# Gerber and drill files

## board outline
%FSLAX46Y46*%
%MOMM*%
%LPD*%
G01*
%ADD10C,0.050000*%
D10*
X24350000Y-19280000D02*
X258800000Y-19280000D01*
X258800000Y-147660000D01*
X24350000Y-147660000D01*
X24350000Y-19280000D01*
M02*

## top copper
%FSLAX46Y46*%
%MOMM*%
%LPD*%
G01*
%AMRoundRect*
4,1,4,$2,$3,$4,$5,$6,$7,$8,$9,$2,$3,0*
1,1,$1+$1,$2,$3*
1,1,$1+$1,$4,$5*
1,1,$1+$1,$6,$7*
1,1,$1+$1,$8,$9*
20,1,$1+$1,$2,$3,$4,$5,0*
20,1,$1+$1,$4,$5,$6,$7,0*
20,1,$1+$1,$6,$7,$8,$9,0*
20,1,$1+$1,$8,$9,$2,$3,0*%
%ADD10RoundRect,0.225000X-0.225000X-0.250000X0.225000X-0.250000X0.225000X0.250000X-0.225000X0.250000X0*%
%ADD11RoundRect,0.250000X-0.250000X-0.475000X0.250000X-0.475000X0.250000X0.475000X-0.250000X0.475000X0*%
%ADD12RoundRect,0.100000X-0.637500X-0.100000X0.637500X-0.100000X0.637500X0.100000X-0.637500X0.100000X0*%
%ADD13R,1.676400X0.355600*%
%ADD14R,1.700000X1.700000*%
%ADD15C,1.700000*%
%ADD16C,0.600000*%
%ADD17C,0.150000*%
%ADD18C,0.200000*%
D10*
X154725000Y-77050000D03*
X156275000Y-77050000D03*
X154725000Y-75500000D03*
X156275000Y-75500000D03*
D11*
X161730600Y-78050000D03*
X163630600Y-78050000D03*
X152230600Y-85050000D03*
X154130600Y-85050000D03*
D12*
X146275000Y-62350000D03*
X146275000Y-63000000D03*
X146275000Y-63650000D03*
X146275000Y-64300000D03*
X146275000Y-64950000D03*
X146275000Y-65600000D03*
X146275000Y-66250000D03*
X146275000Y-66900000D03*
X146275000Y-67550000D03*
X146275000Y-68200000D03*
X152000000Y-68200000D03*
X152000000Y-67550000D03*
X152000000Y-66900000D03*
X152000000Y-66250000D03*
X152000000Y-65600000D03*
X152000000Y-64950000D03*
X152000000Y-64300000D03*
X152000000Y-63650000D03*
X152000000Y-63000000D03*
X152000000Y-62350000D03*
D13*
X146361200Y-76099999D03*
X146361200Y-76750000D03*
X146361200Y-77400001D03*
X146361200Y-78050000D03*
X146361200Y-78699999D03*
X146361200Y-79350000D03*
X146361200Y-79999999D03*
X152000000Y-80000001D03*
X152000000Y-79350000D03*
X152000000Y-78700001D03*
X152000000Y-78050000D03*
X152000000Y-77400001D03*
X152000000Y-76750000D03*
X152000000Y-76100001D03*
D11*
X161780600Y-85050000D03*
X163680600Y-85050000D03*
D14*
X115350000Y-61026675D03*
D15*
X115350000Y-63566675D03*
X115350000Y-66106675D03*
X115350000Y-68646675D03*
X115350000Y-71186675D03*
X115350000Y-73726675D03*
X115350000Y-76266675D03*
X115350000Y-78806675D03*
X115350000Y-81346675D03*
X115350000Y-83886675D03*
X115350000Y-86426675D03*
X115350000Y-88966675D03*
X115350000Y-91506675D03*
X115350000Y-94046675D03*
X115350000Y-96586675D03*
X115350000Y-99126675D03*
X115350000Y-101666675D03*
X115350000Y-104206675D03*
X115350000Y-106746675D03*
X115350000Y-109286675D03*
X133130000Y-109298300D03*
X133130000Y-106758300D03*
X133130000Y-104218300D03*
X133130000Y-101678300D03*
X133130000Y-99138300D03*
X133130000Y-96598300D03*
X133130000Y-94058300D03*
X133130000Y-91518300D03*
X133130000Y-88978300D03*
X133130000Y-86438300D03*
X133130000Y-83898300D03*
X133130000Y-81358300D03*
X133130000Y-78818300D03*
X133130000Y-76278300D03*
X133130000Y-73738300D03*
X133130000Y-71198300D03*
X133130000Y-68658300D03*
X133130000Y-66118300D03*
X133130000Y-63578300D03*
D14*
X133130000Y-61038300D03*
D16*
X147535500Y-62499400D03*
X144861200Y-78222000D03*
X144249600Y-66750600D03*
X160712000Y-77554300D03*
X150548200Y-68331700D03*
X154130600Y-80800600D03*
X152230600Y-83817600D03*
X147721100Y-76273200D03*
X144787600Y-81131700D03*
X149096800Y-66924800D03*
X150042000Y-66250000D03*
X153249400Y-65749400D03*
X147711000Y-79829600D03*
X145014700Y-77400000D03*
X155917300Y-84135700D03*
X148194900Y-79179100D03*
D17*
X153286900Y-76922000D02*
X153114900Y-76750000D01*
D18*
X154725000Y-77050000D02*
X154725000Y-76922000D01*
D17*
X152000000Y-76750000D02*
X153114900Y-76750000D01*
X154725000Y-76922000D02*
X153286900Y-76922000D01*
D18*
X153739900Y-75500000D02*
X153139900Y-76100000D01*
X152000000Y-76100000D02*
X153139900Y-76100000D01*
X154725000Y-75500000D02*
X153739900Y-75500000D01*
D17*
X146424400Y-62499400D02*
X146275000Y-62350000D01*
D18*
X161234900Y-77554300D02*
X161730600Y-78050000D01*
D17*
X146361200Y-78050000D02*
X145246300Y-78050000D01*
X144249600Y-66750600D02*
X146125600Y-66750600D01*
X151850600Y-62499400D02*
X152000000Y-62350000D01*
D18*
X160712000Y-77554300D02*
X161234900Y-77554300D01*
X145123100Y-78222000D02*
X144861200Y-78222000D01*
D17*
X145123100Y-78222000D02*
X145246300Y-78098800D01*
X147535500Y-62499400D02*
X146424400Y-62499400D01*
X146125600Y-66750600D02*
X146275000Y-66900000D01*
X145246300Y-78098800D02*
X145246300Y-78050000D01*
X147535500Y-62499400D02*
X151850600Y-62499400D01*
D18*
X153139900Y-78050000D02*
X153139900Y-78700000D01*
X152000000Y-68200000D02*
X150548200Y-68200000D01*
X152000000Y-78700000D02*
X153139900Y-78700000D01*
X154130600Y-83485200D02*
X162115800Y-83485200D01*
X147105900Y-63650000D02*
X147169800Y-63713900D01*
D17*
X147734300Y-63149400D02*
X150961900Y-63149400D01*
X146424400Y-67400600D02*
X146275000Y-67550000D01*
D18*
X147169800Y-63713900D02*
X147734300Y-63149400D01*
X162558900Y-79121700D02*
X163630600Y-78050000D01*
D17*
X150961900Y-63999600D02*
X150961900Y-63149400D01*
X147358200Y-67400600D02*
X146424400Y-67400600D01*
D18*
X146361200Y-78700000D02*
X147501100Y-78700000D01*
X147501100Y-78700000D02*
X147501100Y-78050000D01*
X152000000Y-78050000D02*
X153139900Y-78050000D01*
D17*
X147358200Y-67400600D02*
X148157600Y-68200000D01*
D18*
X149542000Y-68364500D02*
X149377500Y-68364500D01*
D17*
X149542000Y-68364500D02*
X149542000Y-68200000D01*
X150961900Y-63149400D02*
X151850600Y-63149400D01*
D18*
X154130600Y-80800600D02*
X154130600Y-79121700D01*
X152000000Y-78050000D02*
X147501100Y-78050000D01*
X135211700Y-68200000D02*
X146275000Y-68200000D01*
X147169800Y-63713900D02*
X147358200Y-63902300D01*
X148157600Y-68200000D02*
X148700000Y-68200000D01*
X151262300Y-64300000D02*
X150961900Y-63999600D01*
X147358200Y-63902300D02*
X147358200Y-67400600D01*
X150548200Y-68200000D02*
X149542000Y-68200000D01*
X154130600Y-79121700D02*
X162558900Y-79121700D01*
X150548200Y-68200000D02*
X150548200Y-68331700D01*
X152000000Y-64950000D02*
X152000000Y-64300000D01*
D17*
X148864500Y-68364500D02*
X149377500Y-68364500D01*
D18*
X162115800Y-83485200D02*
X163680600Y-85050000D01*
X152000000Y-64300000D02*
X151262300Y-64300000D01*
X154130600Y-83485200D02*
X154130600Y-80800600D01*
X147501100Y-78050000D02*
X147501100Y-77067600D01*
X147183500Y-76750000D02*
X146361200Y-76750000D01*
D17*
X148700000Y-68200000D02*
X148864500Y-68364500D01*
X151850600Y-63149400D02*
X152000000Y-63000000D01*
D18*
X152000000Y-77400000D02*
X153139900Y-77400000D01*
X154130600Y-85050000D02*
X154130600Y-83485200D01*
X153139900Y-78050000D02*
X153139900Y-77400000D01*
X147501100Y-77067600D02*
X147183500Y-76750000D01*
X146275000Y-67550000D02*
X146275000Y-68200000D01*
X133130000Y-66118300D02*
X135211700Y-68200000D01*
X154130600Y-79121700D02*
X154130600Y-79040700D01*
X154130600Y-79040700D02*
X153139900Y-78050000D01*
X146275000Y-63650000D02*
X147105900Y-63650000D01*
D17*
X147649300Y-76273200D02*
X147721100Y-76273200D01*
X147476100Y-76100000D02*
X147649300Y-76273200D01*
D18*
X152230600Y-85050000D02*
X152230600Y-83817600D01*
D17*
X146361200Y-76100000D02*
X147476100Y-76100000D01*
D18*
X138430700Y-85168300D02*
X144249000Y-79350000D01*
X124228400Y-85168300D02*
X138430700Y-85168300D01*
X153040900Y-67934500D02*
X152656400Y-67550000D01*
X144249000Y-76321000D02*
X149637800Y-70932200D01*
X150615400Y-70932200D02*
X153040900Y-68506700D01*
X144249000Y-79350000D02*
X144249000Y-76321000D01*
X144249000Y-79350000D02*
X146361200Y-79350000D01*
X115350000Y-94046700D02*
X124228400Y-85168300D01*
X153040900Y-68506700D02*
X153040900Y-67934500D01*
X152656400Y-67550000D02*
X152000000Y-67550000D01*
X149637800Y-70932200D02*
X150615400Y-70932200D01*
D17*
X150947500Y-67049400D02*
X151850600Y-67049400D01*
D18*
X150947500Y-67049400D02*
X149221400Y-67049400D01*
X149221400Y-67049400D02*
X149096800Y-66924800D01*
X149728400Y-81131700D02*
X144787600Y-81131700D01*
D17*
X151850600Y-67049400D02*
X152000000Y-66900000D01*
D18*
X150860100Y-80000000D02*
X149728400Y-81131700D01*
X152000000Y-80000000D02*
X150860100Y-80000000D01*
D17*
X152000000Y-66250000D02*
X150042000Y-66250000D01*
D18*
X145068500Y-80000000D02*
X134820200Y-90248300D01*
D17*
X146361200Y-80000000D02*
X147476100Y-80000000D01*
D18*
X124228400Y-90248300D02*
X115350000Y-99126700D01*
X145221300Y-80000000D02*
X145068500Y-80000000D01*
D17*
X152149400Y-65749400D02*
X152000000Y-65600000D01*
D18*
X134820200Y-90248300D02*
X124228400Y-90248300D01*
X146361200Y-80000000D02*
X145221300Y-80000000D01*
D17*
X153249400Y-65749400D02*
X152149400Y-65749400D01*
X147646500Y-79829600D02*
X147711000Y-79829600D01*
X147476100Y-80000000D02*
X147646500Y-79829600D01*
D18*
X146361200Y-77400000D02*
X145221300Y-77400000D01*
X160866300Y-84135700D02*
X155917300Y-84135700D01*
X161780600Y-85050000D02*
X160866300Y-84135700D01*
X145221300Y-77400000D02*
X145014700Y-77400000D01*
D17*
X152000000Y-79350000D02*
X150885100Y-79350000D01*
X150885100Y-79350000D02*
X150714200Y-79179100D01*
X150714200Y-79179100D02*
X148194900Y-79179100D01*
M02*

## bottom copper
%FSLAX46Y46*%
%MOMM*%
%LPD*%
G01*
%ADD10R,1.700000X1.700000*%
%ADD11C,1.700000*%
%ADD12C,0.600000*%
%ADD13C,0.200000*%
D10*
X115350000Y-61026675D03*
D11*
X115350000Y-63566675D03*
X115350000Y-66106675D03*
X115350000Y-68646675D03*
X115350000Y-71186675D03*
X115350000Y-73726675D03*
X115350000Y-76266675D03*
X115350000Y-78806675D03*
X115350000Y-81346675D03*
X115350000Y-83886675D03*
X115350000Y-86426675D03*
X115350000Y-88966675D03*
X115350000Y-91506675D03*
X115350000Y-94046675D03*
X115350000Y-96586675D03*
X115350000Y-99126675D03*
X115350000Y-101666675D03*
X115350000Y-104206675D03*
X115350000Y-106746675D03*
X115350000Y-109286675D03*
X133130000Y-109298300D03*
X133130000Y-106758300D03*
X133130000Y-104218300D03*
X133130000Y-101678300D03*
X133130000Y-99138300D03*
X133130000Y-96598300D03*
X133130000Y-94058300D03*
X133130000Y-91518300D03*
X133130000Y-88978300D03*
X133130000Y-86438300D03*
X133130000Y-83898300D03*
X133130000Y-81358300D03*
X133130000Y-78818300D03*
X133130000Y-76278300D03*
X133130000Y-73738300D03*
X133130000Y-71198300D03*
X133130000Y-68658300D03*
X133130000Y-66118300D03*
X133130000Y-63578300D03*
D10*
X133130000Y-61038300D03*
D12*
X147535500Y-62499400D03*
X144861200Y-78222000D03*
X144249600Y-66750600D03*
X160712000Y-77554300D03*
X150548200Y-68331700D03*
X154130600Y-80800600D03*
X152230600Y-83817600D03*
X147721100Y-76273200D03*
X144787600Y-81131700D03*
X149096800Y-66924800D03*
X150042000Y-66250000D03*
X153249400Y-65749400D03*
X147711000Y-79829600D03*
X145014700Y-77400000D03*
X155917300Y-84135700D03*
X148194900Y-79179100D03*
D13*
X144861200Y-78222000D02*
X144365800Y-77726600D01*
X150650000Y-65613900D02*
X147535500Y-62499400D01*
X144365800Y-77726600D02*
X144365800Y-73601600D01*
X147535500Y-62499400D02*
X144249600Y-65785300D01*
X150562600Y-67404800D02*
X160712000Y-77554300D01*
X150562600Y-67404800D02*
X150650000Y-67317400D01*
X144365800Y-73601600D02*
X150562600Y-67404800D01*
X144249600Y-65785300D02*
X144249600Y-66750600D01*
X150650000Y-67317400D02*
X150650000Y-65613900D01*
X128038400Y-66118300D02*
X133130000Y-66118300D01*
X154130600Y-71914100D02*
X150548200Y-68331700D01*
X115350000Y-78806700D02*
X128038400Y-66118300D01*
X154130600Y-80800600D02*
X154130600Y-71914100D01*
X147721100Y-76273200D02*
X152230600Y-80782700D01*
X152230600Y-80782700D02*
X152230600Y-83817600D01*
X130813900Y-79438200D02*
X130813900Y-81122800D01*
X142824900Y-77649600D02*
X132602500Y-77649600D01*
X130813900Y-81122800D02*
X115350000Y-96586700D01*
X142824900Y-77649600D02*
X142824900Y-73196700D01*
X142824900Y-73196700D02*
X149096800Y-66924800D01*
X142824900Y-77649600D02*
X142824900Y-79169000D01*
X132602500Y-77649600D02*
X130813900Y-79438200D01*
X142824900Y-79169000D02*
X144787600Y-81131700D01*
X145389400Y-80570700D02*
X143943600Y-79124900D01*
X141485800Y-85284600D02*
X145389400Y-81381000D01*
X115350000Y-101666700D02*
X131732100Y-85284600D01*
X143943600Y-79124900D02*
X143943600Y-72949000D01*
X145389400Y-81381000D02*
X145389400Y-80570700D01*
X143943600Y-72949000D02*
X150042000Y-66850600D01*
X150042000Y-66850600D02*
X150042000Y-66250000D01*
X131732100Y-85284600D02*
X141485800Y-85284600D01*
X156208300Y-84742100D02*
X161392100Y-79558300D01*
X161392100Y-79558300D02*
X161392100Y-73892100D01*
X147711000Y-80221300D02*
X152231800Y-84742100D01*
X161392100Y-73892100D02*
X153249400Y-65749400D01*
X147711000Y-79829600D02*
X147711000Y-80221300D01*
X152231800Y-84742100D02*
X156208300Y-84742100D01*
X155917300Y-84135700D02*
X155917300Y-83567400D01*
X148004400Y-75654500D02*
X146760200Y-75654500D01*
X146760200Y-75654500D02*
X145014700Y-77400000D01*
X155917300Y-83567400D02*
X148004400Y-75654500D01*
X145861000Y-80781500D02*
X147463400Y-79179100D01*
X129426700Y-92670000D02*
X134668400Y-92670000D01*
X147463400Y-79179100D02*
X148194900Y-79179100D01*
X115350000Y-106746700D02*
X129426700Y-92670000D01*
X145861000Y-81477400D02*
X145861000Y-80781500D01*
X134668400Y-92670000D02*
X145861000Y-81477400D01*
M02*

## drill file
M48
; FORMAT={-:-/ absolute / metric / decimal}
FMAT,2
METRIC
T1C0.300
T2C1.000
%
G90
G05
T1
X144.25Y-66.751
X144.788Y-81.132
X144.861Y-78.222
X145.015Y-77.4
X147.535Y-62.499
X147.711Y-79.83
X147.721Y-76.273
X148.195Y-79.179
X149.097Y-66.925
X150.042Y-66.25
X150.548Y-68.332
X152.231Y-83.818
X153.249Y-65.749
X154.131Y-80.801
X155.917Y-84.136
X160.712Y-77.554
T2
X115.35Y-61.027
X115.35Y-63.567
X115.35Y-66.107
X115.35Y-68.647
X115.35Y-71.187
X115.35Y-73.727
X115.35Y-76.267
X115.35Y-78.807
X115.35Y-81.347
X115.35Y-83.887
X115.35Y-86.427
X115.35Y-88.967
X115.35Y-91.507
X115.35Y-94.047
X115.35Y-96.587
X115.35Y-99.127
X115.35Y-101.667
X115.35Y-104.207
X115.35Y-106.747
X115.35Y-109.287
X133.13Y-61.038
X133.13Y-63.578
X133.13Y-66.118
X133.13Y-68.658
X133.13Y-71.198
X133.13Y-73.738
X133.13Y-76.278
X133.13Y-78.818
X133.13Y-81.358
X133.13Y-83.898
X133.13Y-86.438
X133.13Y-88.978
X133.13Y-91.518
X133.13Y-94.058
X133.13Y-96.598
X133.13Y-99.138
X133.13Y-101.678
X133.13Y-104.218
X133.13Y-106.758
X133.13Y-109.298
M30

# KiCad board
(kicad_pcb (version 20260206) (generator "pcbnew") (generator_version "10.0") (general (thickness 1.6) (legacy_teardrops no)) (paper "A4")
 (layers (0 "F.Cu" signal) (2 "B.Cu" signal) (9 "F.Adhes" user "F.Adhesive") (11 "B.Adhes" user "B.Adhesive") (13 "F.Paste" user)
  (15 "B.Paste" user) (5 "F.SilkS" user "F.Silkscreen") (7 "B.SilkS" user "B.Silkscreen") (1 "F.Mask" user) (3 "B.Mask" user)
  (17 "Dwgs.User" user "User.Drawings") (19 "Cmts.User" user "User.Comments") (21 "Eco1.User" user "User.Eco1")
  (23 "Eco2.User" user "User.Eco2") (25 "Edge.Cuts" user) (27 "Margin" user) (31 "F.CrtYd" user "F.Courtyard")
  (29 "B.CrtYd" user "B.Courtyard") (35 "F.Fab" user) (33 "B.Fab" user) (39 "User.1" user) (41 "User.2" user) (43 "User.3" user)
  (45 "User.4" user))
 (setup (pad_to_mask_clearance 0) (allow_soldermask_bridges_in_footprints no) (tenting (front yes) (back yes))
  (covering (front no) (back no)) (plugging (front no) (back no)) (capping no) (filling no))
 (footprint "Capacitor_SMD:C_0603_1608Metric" (layer "F.Cu") (at 155.5 77.05)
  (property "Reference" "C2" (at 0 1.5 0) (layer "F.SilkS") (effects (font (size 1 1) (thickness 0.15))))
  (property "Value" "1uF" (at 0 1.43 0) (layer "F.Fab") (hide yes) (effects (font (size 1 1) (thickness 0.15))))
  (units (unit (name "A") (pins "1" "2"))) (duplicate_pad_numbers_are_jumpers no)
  (pad "1" smd roundrect (at -0.775 0) (size 0.9 0.95) (layers "F.Cu" "F.Mask" "F.Paste") (roundrect_rratio 0.25) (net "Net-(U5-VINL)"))
  (pad "2" smd roundrect (at 0.775 0) (size 0.9 0.95) (layers "F.Cu" "F.Mask" "F.Paste") (roundrect_rratio 0.25) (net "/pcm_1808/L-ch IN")))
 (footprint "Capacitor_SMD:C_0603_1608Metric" (layer "F.Cu") (at 155.5 75.5)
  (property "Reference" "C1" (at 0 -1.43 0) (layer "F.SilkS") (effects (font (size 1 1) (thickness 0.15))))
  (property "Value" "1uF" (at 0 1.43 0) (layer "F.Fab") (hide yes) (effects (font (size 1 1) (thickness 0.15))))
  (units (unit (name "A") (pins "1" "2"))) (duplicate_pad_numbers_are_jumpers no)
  (pad "1" smd roundrect (at -0.775 0) (size 0.9 0.95) (layers "F.Cu" "F.Mask" "F.Paste") (roundrect_rratio 0.25) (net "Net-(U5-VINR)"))
  (pad "2" smd roundrect (at 0.775 0) (size 0.9 0.95) (layers "F.Cu" "F.Mask" "F.Paste") (roundrect_rratio 0.25) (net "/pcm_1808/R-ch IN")))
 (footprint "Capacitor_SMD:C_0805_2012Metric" (layer "F.Cu") (at 162.6806 78.05)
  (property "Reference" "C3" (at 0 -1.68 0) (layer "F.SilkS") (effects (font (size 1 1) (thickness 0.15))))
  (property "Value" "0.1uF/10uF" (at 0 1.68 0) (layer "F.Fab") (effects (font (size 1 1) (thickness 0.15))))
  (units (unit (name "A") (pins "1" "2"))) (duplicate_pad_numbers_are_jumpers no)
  (pad "1" smd roundrect (at -0.95 0) (size 1 1.45) (layers "F.Cu" "F.Mask" "F.Paste") (roundrect_rratio 0.25) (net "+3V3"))
  (pad "2" smd roundrect (at 0.95 0) (size 1 1.45) (layers "F.Cu" "F.Mask" "F.Paste") (roundrect_rratio 0.25) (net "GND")))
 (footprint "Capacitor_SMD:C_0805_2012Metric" (layer "F.Cu") (at 153.1806 85.05)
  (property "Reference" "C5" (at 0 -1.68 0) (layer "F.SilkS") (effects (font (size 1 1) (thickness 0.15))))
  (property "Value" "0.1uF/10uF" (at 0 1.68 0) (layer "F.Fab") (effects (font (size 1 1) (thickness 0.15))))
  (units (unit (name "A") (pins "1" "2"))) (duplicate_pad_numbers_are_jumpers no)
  (pad "1" smd roundrect (at -0.95 0) (size 1 1.45) (layers "F.Cu" "F.Mask" "F.Paste") (roundrect_rratio 0.25) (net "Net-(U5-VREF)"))
  (pad "2" smd roundrect (at 0.95 0) (size 1 1.45) (layers "F.Cu" "F.Mask" "F.Paste") (roundrect_rratio 0.25) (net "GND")))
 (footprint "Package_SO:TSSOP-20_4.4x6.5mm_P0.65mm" (layer "F.Cu") (at 149.1375 65.275)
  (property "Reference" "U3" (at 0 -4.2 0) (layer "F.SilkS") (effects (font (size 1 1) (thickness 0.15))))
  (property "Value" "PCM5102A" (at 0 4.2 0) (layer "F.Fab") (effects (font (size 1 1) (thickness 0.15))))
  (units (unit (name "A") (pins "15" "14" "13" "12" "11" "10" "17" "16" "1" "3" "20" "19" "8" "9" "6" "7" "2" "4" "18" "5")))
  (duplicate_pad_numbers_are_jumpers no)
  (pad "1" smd roundrect (at -2.8625 -2.925) (size 1.475 0.4) (layers "F.Cu" "F.Mask" "F.Paste") (roundrect_rratio 0.25) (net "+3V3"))
  (pad "2" smd roundrect (at -2.8625 -2.275) (size 1.475 0.4) (layers "F.Cu" "F.Mask" "F.Paste") (roundrect_rratio 0.25)
   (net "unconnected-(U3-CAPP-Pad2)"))
  (pad "3" smd roundrect (at -2.8625 -1.625) (size 1.475 0.4) (layers "F.Cu" "F.Mask" "F.Paste") (roundrect_rratio 0.25) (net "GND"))
  (pad "4" smd roundrect (at -2.8625 -0.975) (size 1.475 0.4) (layers "F.Cu" "F.Mask" "F.Paste") (roundrect_rratio 0.25)
   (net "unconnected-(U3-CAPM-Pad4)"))
  (pad "5" smd roundrect (at -2.8625 -0.325) (size 1.475 0.4) (layers "F.Cu" "F.Mask" "F.Paste") (roundrect_rratio 0.25) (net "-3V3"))
  (pad "6" smd roundrect (at -2.8625 0.325) (size 1.475 0.4) (layers "F.Cu" "F.Mask" "F.Paste") (roundrect_rratio 0.25)
   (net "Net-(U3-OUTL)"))
  (pad "7" smd roundrect (at -2.8625 0.975) (size 1.475 0.4) (layers "F.Cu" "F.Mask" "F.Paste") (roundrect_rratio 0.25)
   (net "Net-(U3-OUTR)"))
  (pad "8" smd roundrect (at -2.8625 1.625) (size 1.475 0.4) (layers "F.Cu" "F.Mask" "F.Paste") (roundrect_rratio 0.25) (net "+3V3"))
  (pad "9" smd roundrect (at -2.8625 2.275) (size 1.475 0.4) (layers "F.Cu" "F.Mask" "F.Paste") (roundrect_rratio 0.25) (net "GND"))
  (pad "10" smd roundrect (at -2.8625 2.925) (size 1.475 0.4) (layers "F.Cu" "F.Mask" "F.Paste") (roundrect_rratio 0.25) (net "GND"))
  (pad "11" smd roundrect (at 2.8625 2.925) (size 1.475 0.4) (layers "F.Cu" "F.Mask" "F.Paste") (roundrect_rratio 0.25) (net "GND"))
  (pad "12" smd roundrect (at 2.8625 2.275) (size 1.475 0.4) (layers "F.Cu" "F.Mask" "F.Paste") (roundrect_rratio 0.25) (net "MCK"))
  (pad "13" smd roundrect (at 2.8625 1.625) (size 1.475 0.4) (layers "F.Cu" "F.Mask" "F.Paste") (roundrect_rratio 0.25) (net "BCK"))
  (pad "14" smd roundrect (at 2.8625 0.975) (size 1.475 0.4) (layers "F.Cu" "F.Mask" "F.Paste") (roundrect_rratio 0.25) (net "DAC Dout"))
  (pad "15" smd roundrect (at 2.8625 0.325) (size 1.475 0.4) (layers "F.Cu" "F.Mask" "F.Paste") (roundrect_rratio 0.25) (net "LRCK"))
  (pad "16" smd roundrect (at 2.8625 -0.325) (size 1.475 0.4) (layers "F.Cu" "F.Mask" "F.Paste") (roundrect_rratio 0.25) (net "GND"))
  (pad "17" smd roundrect (at 2.8625 -0.975) (size 1.475 0.4) (layers "F.Cu" "F.Mask" "F.Paste") (roundrect_rratio 0.25) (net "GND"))
  (pad "18" smd roundrect (at 2.8625 -1.625) (size 1.475 0.4) (layers "F.Cu" "F.Mask" "F.Paste") (roundrect_rratio 0.25)
   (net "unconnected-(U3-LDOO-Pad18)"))
  (pad "19" smd roundrect (at 2.8625 -2.275) (size 1.475 0.4) (layers "F.Cu" "F.Mask" "F.Paste") (roundrect_rratio 0.25) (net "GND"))
  (pad "20" smd roundrect (at 2.8625 -2.925) (size 1.475 0.4) (layers "F.Cu" "F.Mask" "F.Paste") (roundrect_rratio 0.25) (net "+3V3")))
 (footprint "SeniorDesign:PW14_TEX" (layer "F.Cu") (at 149.1806 78.05)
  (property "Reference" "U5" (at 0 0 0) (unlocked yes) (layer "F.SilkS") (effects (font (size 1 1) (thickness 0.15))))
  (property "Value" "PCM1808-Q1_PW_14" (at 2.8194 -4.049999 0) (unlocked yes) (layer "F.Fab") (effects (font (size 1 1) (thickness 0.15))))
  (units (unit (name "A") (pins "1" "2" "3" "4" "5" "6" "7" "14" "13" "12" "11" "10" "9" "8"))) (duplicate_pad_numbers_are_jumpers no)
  (pad "1" smd rect (at -2.8194 -1.950001) (size 1.6764 0.3556) (layers "F.Cu" "F.Mask" "F.Paste") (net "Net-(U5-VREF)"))
  (pad "2" smd rect (at -2.8194 -1.3) (size 1.6764 0.3556) (layers "F.Cu" "F.Mask" "F.Paste") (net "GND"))
  (pad "3" smd rect (at -2.8194 -0.649999) (size 1.6764 0.3556) (layers "F.Cu" "F.Mask" "F.Paste") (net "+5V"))
  (pad "4" smd rect (at -2.8194 0) (size 1.6764 0.3556) (layers "F.Cu" "F.Mask" "F.Paste") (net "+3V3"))
  (pad "5" smd rect (at -2.8194 0.649999) (size 1.6764 0.3556) (layers "F.Cu" "F.Mask" "F.Paste") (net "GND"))
  (pad "6" smd rect (at -2.8194 1.3) (size 1.6764 0.3556) (layers "F.Cu" "F.Mask" "F.Paste") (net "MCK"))
  (pad "7" smd rect (at -2.8194 1.949999) (size 1.6764 0.3556) (layers "F.Cu" "F.Mask" "F.Paste") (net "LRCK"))
  (pad "8" smd rect (at 2.8194 1.950001) (size 1.6764 0.3556) (layers "F.Cu" "F.Mask" "F.Paste") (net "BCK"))
  (pad "9" smd rect (at 2.8194 1.3) (size 1.6764 0.3556) (layers "F.Cu" "F.Mask" "F.Paste") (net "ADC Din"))
  (pad "10" smd rect (at 2.8194 0.650001) (size 1.6764 0.3556) (layers "F.Cu" "F.Mask" "F.Paste") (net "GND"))
  (pad "11" smd rect (at 2.8194 0) (size 1.6764 0.3556) (layers "F.Cu" "F.Mask" "F.Paste") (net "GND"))
  (pad "12" smd rect (at 2.8194 -0.649999) (size 1.6764 0.3556) (layers "F.Cu" "F.Mask" "F.Paste") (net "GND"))
  (pad "13" smd rect (at 2.8194 -1.3) (size 1.6764 0.3556) (layers "F.Cu" "F.Mask" "F.Paste") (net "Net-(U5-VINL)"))
  (pad "14" smd rect (at 2.8194 -1.949999) (size 1.6764 0.3556) (layers "F.Cu" "F.Mask" "F.Paste") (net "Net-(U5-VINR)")))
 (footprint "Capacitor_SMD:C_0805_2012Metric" (layer "F.Cu") (at 162.7306 85.05)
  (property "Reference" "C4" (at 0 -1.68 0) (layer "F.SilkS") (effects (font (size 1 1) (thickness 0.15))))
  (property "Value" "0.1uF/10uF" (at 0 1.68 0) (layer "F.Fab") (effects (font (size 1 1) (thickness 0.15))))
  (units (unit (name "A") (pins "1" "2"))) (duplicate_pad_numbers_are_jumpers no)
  (pad "1" smd roundrect (at -0.95 0) (size 1 1.45) (layers "F.Cu" "F.Mask" "F.Paste") (roundrect_rratio 0.25) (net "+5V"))
  (pad "2" smd roundrect (at 0.95 0) (size 1 1.45) (layers "F.Cu" "F.Mask" "F.Paste") (roundrect_rratio 0.25) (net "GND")))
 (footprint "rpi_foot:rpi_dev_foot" (layer "F.Cu") (at 133.13 61.7383)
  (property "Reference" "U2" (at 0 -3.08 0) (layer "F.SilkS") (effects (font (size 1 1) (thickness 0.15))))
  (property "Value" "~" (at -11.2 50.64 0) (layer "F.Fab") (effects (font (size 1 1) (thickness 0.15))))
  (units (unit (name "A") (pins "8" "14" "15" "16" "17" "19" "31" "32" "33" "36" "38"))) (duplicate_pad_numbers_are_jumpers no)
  (pad "1" thru_hole rect (at -17.78 -0.711625) (size 1.7 1.7) (drill 1) (layers "*.Cu" "*.Mask") (remove_unused_layers no))
  (pad "2" thru_hole circle (at -17.78 1.828375) (size 1.7 1.7) (drill 1) (layers "*.Cu" "*.Mask") (remove_unused_layers no))
  (pad "3" thru_hole circle (at -17.78 4.368375) (size 1.7 1.7) (drill 1) (layers "*.Cu" "*.Mask") (remove_unused_layers no))
  (pad "4" thru_hole circle (at -17.78 6.908375) (size 1.7 1.7) (drill 1) (layers "*.Cu" "*.Mask") (remove_unused_layers no))
  (pad "5" thru_hole circle (at -17.78 9.448375) (size 1.7 1.7) (drill 1) (layers "*.Cu" "*.Mask") (remove_unused_layers no))
  (pad "6" thru_hole circle (at -17.78 11.988375) (size 1.7 1.7) (drill 1) (layers "*.Cu" "*.Mask") (remove_unused_layers no))
  (pad "7" thru_hole circle (at -17.78 14.528375) (size 1.7 1.7) (drill 1) (layers "*.Cu" "*.Mask") (remove_unused_layers no))
  (pad "8" thru_hole circle (at -17.78 17.068375) (size 1.7 1.7) (drill 1) (layers "*.Cu" "*.Mask") (remove_unused_layers no) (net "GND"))
  (pad "9" thru_hole circle (at -17.78 19.608375) (size 1.7 1.7) (drill 1) (layers "*.Cu" "*.Mask") (remove_unused_layers no))
  (pad "10" thru_hole circle (at -17.78 22.148375) (size 1.7 1.7) (drill 1) (layers "*.Cu" "*.Mask") (remove_unused_layers no))
  (pad "11" thru_hole circle (at -17.78 24.688375) (size 1.7 1.7) (drill 1) (layers "*.Cu" "*.Mask") (remove_unused_layers no))
  (pad "12" thru_hole circle (at -17.78 27.228375) (size 1.7 1.7) (drill 1) (layers "*.Cu" "*.Mask") (remove_unused_layers no))
  (pad "13" thru_hole circle (at -17.78 29.768375) (size 1.7 1.7) (drill 1) (layers "*.Cu" "*.Mask") (remove_unused_layers no))
  (pad "14" thru_hole circle (at -17.78 32.308375) (size 1.7 1.7) (drill 1) (layers "*.Cu" "*.Mask") (remove_unused_layers no) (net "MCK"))
  (pad "15" thru_hole circle (at -17.78 34.848375) (size 1.7 1.7) (drill 1) (layers "*.Cu" "*.Mask") (remove_unused_layers no) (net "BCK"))
  (pad "16" thru_hole circle (at -17.78 37.388375) (size 1.7 1.7) (drill 1) (layers "*.Cu" "*.Mask") (remove_unused_layers no) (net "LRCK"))
  (pad "17" thru_hole circle (at -17.78 39.928375) (size 1.7 1.7) (drill 1) (layers "*.Cu" "*.Mask") (remove_unused_layers no)
   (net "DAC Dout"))
  (pad "18" thru_hole circle (at -17.78 42.468375) (size 1.7 1.7) (drill 1) (layers "*.Cu" "*.Mask") (remove_unused_layers no))
  (pad "19" thru_hole circle (at -17.78 45.008375) (size 1.7 1.7) (drill 1) (layers "*.Cu" "*.Mask") (remove_unused_layers no)
   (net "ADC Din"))
  (pad "20" thru_hole circle (at -17.78 47.548375) (size 1.7 1.7) (drill 1) (layers "*.Cu" "*.Mask") (remove_unused_layers no))
  (pad "21" thru_hole circle (at 0 47.56) (size 1.7 1.7) (drill 1) (layers "*.Cu" "*.Mask") (remove_unused_layers no))
  (pad "22" thru_hole circle (at 0 45.02) (size 1.7 1.7) (drill 1) (layers "*.Cu" "*.Mask") (remove_unused_layers no))
  (pad "23" thru_hole circle (at 0 42.48) (size 1.7 1.7) (drill 1) (layers "*.Cu" "*.Mask") (remove_unused_layers no))
  (pad "24" thru_hole circle (at 0 39.94) (size 1.7 1.7) (drill 1) (layers "*.Cu" "*.Mask") (remove_unused_layers no))
  (pad "25" thru_hole circle (at 0 37.4) (size 1.7 1.7) (drill 1) (layers "*.Cu" "*.Mask") (remove_unused_layers no))
  (pad "26" thru_hole circle (at 0 34.86) (size 1.7 1.7) (drill 1) (layers "*.Cu" "*.Mask") (remove_unused_layers no))
  (pad "27" thru_hole circle (at 0 32.32) (size 1.7 1.7) (drill 1) (layers "*.Cu" "*.Mask") (remove_unused_layers no))
  (pad "28" thru_hole circle (at 0 29.78) (size 1.7 1.7) (drill 1) (layers "*.Cu" "*.Mask") (remove_unused_layers no))
  (pad "29" thru_hole circle (at 0 27.24) (size 1.7 1.7) (drill 1) (layers "*.Cu" "*.Mask") (remove_unused_layers no))
  (pad "30" thru_hole circle (at 0 24.7) (size 1.7 1.7) (drill 1) (layers "*.Cu" "*.Mask") (remove_unused_layers no))
  (pad "31" thru_hole circle (at 0 22.16) (size 1.7 1.7) (drill 1) (layers "*.Cu" "*.Mask") (remove_unused_layers no) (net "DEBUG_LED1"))
  (pad "32" thru_hole circle (at 0 19.62) (size 1.7 1.7) (drill 1) (layers "*.Cu" "*.Mask") (remove_unused_layers no) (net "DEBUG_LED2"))
  (pad "33" thru_hole circle (at 0 17.08) (size 1.7 1.7) (drill 1) (layers "*.Cu" "*.Mask") (remove_unused_layers no) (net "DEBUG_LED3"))
  (pad "34" thru_hole circle (at 0 14.54) (size 1.7 1.7) (drill 1) (layers "*.Cu" "*.Mask") (remove_unused_layers no))
  (pad "35" thru_hole circle (at 0 12) (size 1.7 1.7) (drill 1) (layers "*.Cu" "*.Mask") (remove_unused_layers no))
  (pad "36" thru_hole circle (at 0 9.46) (size 1.7 1.7) (drill 1) (layers "*.Cu" "*.Mask") (remove_unused_layers no) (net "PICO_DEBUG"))
  (pad "37" thru_hole circle (at 0 6.92) (size 1.7 1.7) (drill 1) (layers "*.Cu" "*.Mask") (remove_unused_layers no))
  (pad "38" thru_hole circle (at 0 4.38) (size 1.7 1.7) (drill 1) (layers "*.Cu" "*.Mask") (remove_unused_layers no) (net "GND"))
  (pad "39" thru_hole circle (at 0 1.84) (size 1.7 1.7) (drill 1) (layers "*.Cu" "*.Mask") (remove_unused_layers no))
  (pad "40" thru_hole rect (at 0 -0.7) (size 1.7 1.7) (drill 1) (layers "*.Cu" "*.Mask") (remove_unused_layers no)))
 (gr_rect (start 24.35 19.28) (end 258.8 147.66) (stroke (width 0.05) (type default)) (fill no) (layer "Edge.Cuts"))
 (segment (start 153.2869 76.922) (end 153.1149 76.75) (width 0.15) (layer "F.Cu") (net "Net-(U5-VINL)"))
 (segment (start 154.725 77.05) (end 154.725 76.922) (width 0.2) (layer "F.Cu") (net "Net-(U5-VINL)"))
 (segment (start 152 76.75) (end 153.1149 76.75) (width 0.15) (layer "F.Cu") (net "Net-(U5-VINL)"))
 (segment (start 154.725 76.922) (end 153.2869 76.922) (width 0.15) (layer "F.Cu") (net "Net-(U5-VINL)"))
 (segment (start 153.7399 75.5) (end 153.1399 76.1) (width 0.2) (layer "F.Cu") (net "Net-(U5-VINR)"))
 (segment (start 152 76.1) (end 153.1399 76.1) (width 0.2) (layer "F.Cu") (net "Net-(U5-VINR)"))
 (segment (start 154.725 75.5) (end 153.7399 75.5) (width 0.2) (layer "F.Cu") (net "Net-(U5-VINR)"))
 (segment (start 146.4244 62.4994) (end 146.275 62.35) (width 0.15) (layer "F.Cu") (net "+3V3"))
 (segment (start 161.2349 77.5543) (end 161.7306 78.05) (width 0.2) (layer "F.Cu") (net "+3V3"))
 (segment (start 146.3612 78.05) (end 145.2463 78.05) (width 0.15) (layer "F.Cu") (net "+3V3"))
 (segment (start 144.2496 66.7506) (end 146.1256 66.7506) (width 0.15) (layer "F.Cu") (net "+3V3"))
 (segment (start 151.8506 62.4994) (end 152 62.35) (width 0.15) (layer "F.Cu") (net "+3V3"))
 (segment (start 160.712 77.5543) (end 161.2349 77.5543) (width 0.2) (layer "F.Cu") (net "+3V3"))
 (segment (start 145.1231 78.222) (end 144.8612 78.222) (width 0.2) (layer "F.Cu") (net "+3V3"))
 (segment (start 145.1231 78.222) (end 145.2463 78.0988) (width 0.15) (layer "F.Cu") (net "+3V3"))
 (segment (start 147.5355 62.4994) (end 146.4244 62.4994) (width 0.15) (layer "F.Cu") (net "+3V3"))
 (segment (start 146.1256 66.7506) (end 146.275 66.9) (width 0.15) (layer "F.Cu") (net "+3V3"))
 (segment (start 145.2463 78.0988) (end 145.2463 78.05) (width 0.15) (layer "F.Cu") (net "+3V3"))
 (segment (start 147.5355 62.4994) (end 151.8506 62.4994) (width 0.15) (layer "F.Cu") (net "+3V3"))
 (via (at 147.5355 62.4994) (size 0.6) (drill 0.3) (layers "F.Cu" "B.Cu") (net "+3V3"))
 (via (at 144.8612 78.222) (size 0.6) (drill 0.3) (layers "F.Cu" "B.Cu") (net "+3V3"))
 (via (at 144.2496 66.7506) (size 0.6) (drill 0.3) (layers "F.Cu" "B.Cu") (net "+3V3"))
 (via (at 160.712 77.5543) (size 0.6) (drill 0.3) (layers "F.Cu" "B.Cu") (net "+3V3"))
 (segment (start 144.8612 78.222) (end 144.3658 77.7266) (width 0.2) (layer "B.Cu") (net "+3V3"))
 (segment (start 150.65 65.6139) (end 147.5355 62.4994) (width 0.2) (layer "B.Cu") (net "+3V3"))
 (segment (start 144.3658 77.7266) (end 144.3658 73.6016) (width 0.2) (layer "B.Cu") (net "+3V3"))
 (segment (start 147.5355 62.4994) (end 144.2496 65.7853) (width 0.2) (layer "B.Cu") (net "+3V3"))
 (segment (start 150.5626 67.4048) (end 160.712 77.5543) (width 0.2) (layer "B.Cu") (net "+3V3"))
 (segment (start 150.5626 67.4048) (end 150.65 67.3174) (width 0.2) (layer "B.Cu") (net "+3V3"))
 (segment (start 144.3658 73.6016) (end 150.5626 67.4048) (width 0.2) (layer "B.Cu") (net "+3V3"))
 (segment (start 144.2496 65.7853) (end 144.2496 66.7506) (width 0.2) (layer "B.Cu") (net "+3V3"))
 (segment (start 150.65 67.3174) (end 150.65 65.6139) (width 0.2) (layer "B.Cu") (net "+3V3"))
 (segment (start 153.1399 78.05) (end 153.1399 78.7) (width 0.2) (layer "F.Cu") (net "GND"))
 (segment (start 152 68.2) (end 150.5482 68.2) (width 0.2) (layer "F.Cu") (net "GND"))
 (segment (start 152 78.7) (end 153.1399 78.7) (width 0.2) (layer "F.Cu") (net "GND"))
 (segment (start 154.1306 83.4852) (end 162.1158 83.4852) (width 0.2) (layer "F.Cu") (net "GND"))
 (segment (start 147.1059 63.65) (end 147.1698 63.7139) (width 0.2) (layer "F.Cu") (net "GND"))
 (segment (start 147.7343 63.1494) (end 150.9619 63.1494) (width 0.15) (layer "F.Cu") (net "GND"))
 (segment (start 146.4244 67.4006) (end 146.275 67.55) (width 0.15) (layer "F.Cu") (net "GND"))
 (segment (start 147.1698 63.7139) (end 147.7343 63.1494) (width 0.2) (layer "F.Cu") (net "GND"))
 (segment (start 162.5589 79.1217) (end 163.6306 78.05) (width 0.2) (layer "F.Cu") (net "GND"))
 (segment (start 150.9619 63.9996) (end 150.9619 63.1494) (width 0.15) (layer "F.Cu") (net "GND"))
 (segment (start 147.3582 67.4006) (end 146.4244 67.4006) (width 0.15) (layer "F.Cu") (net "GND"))
 (segment (start 146.3612 78.7) (end 147.5011 78.7) (width 0.2) (layer "F.Cu") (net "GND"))
 (segment (start 147.5011 78.7) (end 147.5011 78.05) (width 0.2) (layer "F.Cu") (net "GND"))
 (segment (start 152 78.05) (end 153.1399 78.05) (width 0.2) (layer "F.Cu") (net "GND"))
 (segment (start 147.3582 67.4006) (end 148.1576 68.2) (width 0.15) (layer "F.Cu") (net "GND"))
 (segment (start 149.542 68.3645) (end 149.3775 68.3645) (width 0.2) (layer "F.Cu") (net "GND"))
 (segment (start 149.542 68.3645) (end 149.542 68.2) (width 0.15) (layer "F.Cu") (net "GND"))
 (segment (start 150.9619 63.1494) (end 151.8506 63.1494) (width 0.15) (layer "F.Cu") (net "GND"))
 (segment (start 154.1306 80.8006) (end 154.1306 79.1217) (width 0.2) (layer "F.Cu") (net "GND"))
 (segment (start 152 78.05) (end 147.5011 78.05) (width 0.2) (layer "F.Cu") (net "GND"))
 (segment (start 135.2117 68.2) (end 146.275 68.2) (width 0.2) (layer "F.Cu") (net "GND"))
 (segment (start 147.1698 63.7139) (end 147.3582 63.9023) (width 0.2) (layer "F.Cu") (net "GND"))
 (segment (start 148.1576 68.2) (end 148.7 68.2) (width 0.2) (layer "F.Cu") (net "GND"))
 (segment (start 151.2623 64.3) (end 150.9619 63.9996) (width 0.2) (layer "F.Cu") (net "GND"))
 (segment (start 147.3582 63.9023) (end 147.3582 67.4006) (width 0.2) (layer "F.Cu") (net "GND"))
 (segment (start 150.5482 68.2) (end 149.542 68.2) (width 0.2) (layer "F.Cu") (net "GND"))
 (segment (start 154.1306 79.1217) (end 162.5589 79.1217) (width 0.2) (layer "F.Cu") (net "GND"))
 (segment (start 150.5482 68.2) (end 150.5482 68.3317) (width 0.2) (layer "F.Cu") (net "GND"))
 (segment (start 152 64.95) (end 152 64.3) (width 0.2) (layer "F.Cu") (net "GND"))
 (segment (start 148.8645 68.3645) (end 149.3775 68.3645) (width 0.15) (layer "F.Cu") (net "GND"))
 (segment (start 162.1158 83.4852) (end 163.6806 85.05) (width 0.2) (layer "F.Cu") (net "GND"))
 (segment (start 152 64.3) (end 151.2623 64.3) (width 0.2) (layer "F.Cu") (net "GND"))
 (segment (start 154.1306 83.4852) (end 154.1306 80.8006) (width 0.2) (layer "F.Cu") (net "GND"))
 (segment (start 147.5011 78.05) (end 147.5011 77.0676) (width 0.2) (layer "F.Cu") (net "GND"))
 (segment (start 147.1835 76.75) (end 146.3612 76.75) (width 0.2) (layer "F.Cu") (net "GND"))
 (segment (start 148.7 68.2) (end 148.8645 68.3645) (width 0.15) (layer "F.Cu") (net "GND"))
 (segment (start 151.8506 63.1494) (end 152 63) (width 0.15) (layer "F.Cu") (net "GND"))
 (segment (start 152 77.4) (end 153.1399 77.4) (width 0.2) (layer "F.Cu") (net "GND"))
 (segment (start 154.1306 85.05) (end 154.1306 83.4852) (width 0.2) (layer "F.Cu") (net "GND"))
 (segment (start 153.1399 78.05) (end 153.1399 77.4) (width 0.2) (layer "F.Cu") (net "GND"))
 (segment (start 147.5011 77.0676) (end 147.1835 76.75) (width 0.2) (layer "F.Cu") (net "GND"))
 (segment (start 146.275 67.55) (end 146.275 68.2) (width 0.2) (layer "F.Cu") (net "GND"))
 (segment (start 133.13 66.1183) (end 135.2117 68.2) (width 0.2) (layer "F.Cu") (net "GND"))
 (segment (start 154.1306 79.1217) (end 154.1306 79.0407) (width 0.2) (layer "F.Cu") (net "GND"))
 (segment (start 154.1306 79.0407) (end 153.1399 78.05) (width 0.2) (layer "F.Cu") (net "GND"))
 (segment (start 146.275 63.65) (end 147.1059 63.65) (width 0.2) (layer "F.Cu") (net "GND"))
 (via (at 150.5482 68.3317) (size 0.6) (drill 0.3) (layers "F.Cu" "B.Cu") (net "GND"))
 (via (at 154.1306 80.8006) (size 0.6) (drill 0.3) (layers "F.Cu" "B.Cu") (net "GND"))
 (segment (start 128.0384 66.1183) (end 133.13 66.1183) (width 0.2) (layer "B.Cu") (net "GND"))
 (segment (start 154.1306 71.9141) (end 150.5482 68.3317) (width 0.2) (layer "B.Cu") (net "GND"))
 (segment (start 115.35 78.8067) (end 128.0384 66.1183) (width 0.2) (layer "B.Cu") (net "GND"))
 (segment (start 154.1306 80.8006) (end 154.1306 71.9141) (width 0.2) (layer "B.Cu") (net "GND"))
 (segment (start 147.6493 76.2732) (end 147.7211 76.2732) (width 0.15) (layer "F.Cu") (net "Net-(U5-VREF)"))
 (segment (start 147.4761 76.1) (end 147.6493 76.2732) (width 0.15) (layer "F.Cu") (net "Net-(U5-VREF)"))
 (segment (start 152.2306 85.05) (end 152.2306 83.8176) (width 0.2) (layer "F.Cu") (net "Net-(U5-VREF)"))
 (segment (start 146.3612 76.1) (end 147.4761 76.1) (width 0.15) (layer "F.Cu") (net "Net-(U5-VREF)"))
 (via (at 152.2306 83.8176) (size 0.6) (drill 0.3) (layers "F.Cu" "B.Cu") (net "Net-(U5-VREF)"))
 (via (at 147.7211 76.2732) (size 0.6) (drill 0.3) (layers "F.Cu" "B.Cu") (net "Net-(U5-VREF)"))
 (segment (start 147.7211 76.2732) (end 152.2306 80.7827) (width 0.2) (layer "B.Cu") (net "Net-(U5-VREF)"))
 (segment (start 152.2306 80.7827) (end 152.2306 83.8176) (width 0.2) (layer "B.Cu") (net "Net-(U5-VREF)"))
 (segment (start 138.4307 85.1683) (end 144.249 79.35) (width 0.2) (layer "F.Cu") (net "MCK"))
 (segment (start 124.2284 85.1683) (end 138.4307 85.1683) (width 0.2) (layer "F.Cu") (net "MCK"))
 (segment (start 153.0409 67.9345) (end 152.6564 67.55) (width 0.2) (layer "F.Cu") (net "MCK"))
 (segment (start 144.249 76.321) (end 149.6378 70.9322) (width 0.2) (layer "F.Cu") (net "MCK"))
 (segment (start 150.6154 70.9322) (end 153.0409 68.5067) (width 0.2) (layer "F.Cu") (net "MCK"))
 (segment (start 144.249 79.35) (end 144.249 76.321) (width 0.2) (layer "F.Cu") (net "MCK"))
 (segment (start 144.249 79.35) (end 146.3612 79.35) (width 0.2) (layer "F.Cu") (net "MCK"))
 (segment (start 115.35 94.0467) (end 124.2284 85.1683) (width 0.2) (layer "F.Cu") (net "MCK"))
 (segment (start 153.0409 68.5067) (end 153.0409 67.9345) (width 0.2) (layer "F.Cu") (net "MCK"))
 (segment (start 152.6564 67.55) (end 152 67.55) (width 0.2) (layer "F.Cu") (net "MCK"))
 (segment (start 149.6378 70.9322) (end 150.6154 70.9322) (width 0.2) (layer "F.Cu") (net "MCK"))
 (segment (start 150.9475 67.0494) (end 151.8506 67.0494) (width 0.15) (layer "F.Cu") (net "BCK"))
 (segment (start 150.9475 67.0494) (end 149.2214 67.0494) (width 0.2) (layer "F.Cu") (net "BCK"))
 (segment (start 149.2214 67.0494) (end 149.0968 66.9248) (width 0.2) (layer "F.Cu") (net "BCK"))
 (segment (start 149.7284 81.1317) (end 144.7876 81.1317) (width 0.2) (layer "F.Cu") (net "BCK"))
 (segment (start 151.8506 67.0494) (end 152 66.9) (width 0.15) (layer "F.Cu") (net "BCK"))
 (segment (start 150.8601 80) (end 149.7284 81.1317) (width 0.2) (layer "F.Cu") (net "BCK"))
 (segment (start 152 80) (end 150.8601 80) (width 0.2) (layer "F.Cu") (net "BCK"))
 (via (at 144.7876 81.1317) (size 0.6) (drill 0.3) (layers "F.Cu" "B.Cu") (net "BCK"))
 (via (at 149.0968 66.9248) (size 0.6) (drill 0.3) (layers "F.Cu" "B.Cu") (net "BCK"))
 (segment (start 130.8139 79.4382) (end 130.8139 81.1228) (width 0.2) (layer "B.Cu") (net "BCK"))
 (segment (start 142.8249 77.6496) (end 132.6025 77.6496) (width 0.2) (layer "B.Cu") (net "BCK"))
 (segment (start 130.8139 81.1228) (end 115.35 96.5867) (width 0.2) (layer "B.Cu") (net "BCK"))
 (segment (start 142.8249 77.6496) (end 142.8249 73.1967) (width 0.2) (layer "B.Cu") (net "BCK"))
 (segment (start 142.8249 73.1967) (end 149.0968 66.9248) (width 0.2) (layer "B.Cu") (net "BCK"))
 (segment (start 142.8249 77.6496) (end 142.8249 79.169) (width 0.2) (layer "B.Cu") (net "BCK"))
 (segment (start 132.6025 77.6496) (end 130.8139 79.4382) (width 0.2) (layer "B.Cu") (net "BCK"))
 (segment (start 142.8249 79.169) (end 144.7876 81.1317) (width 0.2) (layer "B.Cu") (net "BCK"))
 (segment (start 152 66.25) (end 150.042 66.25) (width 0.15) (layer "F.Cu") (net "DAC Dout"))
 (via (at 150.042 66.25) (size 0.6) (drill 0.3) (layers "F.Cu" "B.Cu") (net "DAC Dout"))
 (segment (start 145.3894 80.5707) (end 143.9436 79.1249) (width 0.2) (layer "B.Cu") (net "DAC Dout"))
 (segment (start 141.4858 85.2846) (end 145.3894 81.381) (width 0.2) (layer "B.Cu") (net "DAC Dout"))
 (segment (start 115.35 101.6667) (end 131.7321 85.2846) (width 0.2) (layer "B.Cu") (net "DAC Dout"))
 (segment (start 143.9436 79.1249) (end 143.9436 72.949) (width 0.2) (layer "B.Cu") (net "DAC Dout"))
 (segment (start 145.3894 81.381) (end 145.3894 80.5707) (width 0.2) (layer "B.Cu") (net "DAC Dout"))
 (segment (start 143.9436 72.949) (end 150.042 66.8506) (width 0.2) (layer "B.Cu") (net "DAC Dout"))
 (segment (start 150.042 66.8506) (end 150.042 66.25) (width 0.2) (layer "B.Cu") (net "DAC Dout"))
 (segment (start 131.7321 85.2846) (end 141.4858 85.2846) (width 0.2) (layer "B.Cu") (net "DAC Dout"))
 (segment (start 145.0685 80) (end 134.8202 90.2483) (width 0.2) (layer "F.Cu") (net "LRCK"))
 (segment (start 146.3612 80) (end 147.4761 80) (width 0.15) (layer "F.Cu") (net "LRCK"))
 (segment (start 124.2284 90.2483) (end 115.35 99.1267) (width 0.2) (layer "F.Cu") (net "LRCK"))
 (segment (start 145.2213 80) (end 145.0685 80) (width 0.2) (layer "F.Cu") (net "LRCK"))
 (segment (start 152.1494 65.7494) (end 152 65.6) (width 0.15) (layer "F.Cu") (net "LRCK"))
 (segment (start 134.8202 90.2483) (end 124.2284 90.2483) (width 0.2) (layer "F.Cu") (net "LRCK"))
 (segment (start 146.3612 80) (end 145.2213 80) (width 0.2) (layer "F.Cu") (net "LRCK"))
 (segment (start 153.2494 65.7494) (end 152.1494 65.7494) (width 0.15) (layer "F.Cu") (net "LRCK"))
 (segment (start 147.6465 79.8296) (end 147.711 79.8296) (width 0.15) (layer "F.Cu") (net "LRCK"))
 (segment (start 147.4761 80) (end 147.6465 79.8296) (width 0.15) (layer "F.Cu") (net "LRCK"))
 (via (at 153.2494 65.7494) (size 0.6) (drill 0.3) (layers "F.Cu" "B.Cu") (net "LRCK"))
 (via (at 147.711 79.8296) (size 0.6) (drill 0.3) (layers "F.Cu" "B.Cu") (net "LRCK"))
 (segment (start 156.2083 84.7421) (end 161.3921 79.5583) (width 0.2) (layer "B.Cu") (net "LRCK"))
 (segment (start 161.3921 79.5583) (end 161.3921 73.8921) (width 0.2) (layer "B.Cu") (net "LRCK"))
 (segment (start 147.711 80.2213) (end 152.2318 84.7421) (width 0.2) (layer "B.Cu") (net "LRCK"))
 (segment (start 161.3921 73.8921) (end 153.2494 65.7494) (width 0.2) (layer "B.Cu") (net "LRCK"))
 (segment (start 147.711 79.8296) (end 147.711 80.2213) (width 0.2) (layer "B.Cu") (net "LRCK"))
 (segment (start 152.2318 84.7421) (end 156.2083 84.7421) (width 0.2) (layer "B.Cu") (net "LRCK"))
 (segment (start 146.3612 77.4) (end 145.2213 77.4) (width 0.2) (layer "F.Cu") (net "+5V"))
 (segment (start 160.8663 84.1357) (end 155.9173 84.1357) (width 0.2) (layer "F.Cu") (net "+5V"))
 (segment (start 161.7806 85.05) (end 160.8663 84.1357) (width 0.2) (layer "F.Cu") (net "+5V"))
 (segment (start 145.2213 77.4) (end 145.0147 77.4) (width 0.2) (layer "F.Cu") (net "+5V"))
 (via (at 145.0147 77.4) (size 0.6) (drill 0.3) (layers "F.Cu" "B.Cu") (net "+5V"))
 (via (at 155.9173 84.1357) (size 0.6) (drill 0.3) (layers "F.Cu" "B.Cu") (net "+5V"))
 (segment (start 155.9173 84.1357) (end 155.9173 83.5674) (width 0.2) (layer "B.Cu") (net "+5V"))
 (segment (start 148.0044 75.6545) (end 146.7602 75.6545) (width 0.2) (layer "B.Cu") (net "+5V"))
 (segment (start 146.7602 75.6545) (end 145.0147 77.4) (width 0.2) (layer "B.Cu") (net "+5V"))
 (segment (start 155.9173 83.5674) (end 148.0044 75.6545) (width 0.2) (layer "B.Cu") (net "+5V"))
 (segment (start 152 79.35) (end 150.8851 79.35) (width 0.15) (layer "F.Cu") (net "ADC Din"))
 (segment (start 150.8851 79.35) (end 150.7142 79.1791) (width 0.15) (layer "F.Cu") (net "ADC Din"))
 (segment (start 150.7142 79.1791) (end 148.1949 79.1791) (width 0.15) (layer "F.Cu") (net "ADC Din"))
 (via (at 148.1949 79.1791) (size 0.6) (drill 0.3) (layers "F.Cu" "B.Cu") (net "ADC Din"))
 (segment (start 145.861 80.7815) (end 147.4634 79.1791) (width 0.2) (layer "B.Cu") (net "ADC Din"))
 (segment (start 129.4267 92.67) (end 134.6684 92.67) (width 0.2) (layer "B.Cu") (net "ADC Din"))
 (segment (start 147.4634 79.1791) (end 148.1949 79.1791) (width 0.2) (layer "B.Cu") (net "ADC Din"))
 (segment (start 115.35 106.7467) (end 129.4267 92.67) (width 0.2) (layer "B.Cu") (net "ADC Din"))
 (segment (start 145.861 81.4774) (end 145.861 80.7815) (width 0.2) (layer "B.Cu") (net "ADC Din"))
 (segment (start 134.6684 92.67) (end 145.861 81.4774) (width 0.2) (layer "B.Cu") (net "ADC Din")))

